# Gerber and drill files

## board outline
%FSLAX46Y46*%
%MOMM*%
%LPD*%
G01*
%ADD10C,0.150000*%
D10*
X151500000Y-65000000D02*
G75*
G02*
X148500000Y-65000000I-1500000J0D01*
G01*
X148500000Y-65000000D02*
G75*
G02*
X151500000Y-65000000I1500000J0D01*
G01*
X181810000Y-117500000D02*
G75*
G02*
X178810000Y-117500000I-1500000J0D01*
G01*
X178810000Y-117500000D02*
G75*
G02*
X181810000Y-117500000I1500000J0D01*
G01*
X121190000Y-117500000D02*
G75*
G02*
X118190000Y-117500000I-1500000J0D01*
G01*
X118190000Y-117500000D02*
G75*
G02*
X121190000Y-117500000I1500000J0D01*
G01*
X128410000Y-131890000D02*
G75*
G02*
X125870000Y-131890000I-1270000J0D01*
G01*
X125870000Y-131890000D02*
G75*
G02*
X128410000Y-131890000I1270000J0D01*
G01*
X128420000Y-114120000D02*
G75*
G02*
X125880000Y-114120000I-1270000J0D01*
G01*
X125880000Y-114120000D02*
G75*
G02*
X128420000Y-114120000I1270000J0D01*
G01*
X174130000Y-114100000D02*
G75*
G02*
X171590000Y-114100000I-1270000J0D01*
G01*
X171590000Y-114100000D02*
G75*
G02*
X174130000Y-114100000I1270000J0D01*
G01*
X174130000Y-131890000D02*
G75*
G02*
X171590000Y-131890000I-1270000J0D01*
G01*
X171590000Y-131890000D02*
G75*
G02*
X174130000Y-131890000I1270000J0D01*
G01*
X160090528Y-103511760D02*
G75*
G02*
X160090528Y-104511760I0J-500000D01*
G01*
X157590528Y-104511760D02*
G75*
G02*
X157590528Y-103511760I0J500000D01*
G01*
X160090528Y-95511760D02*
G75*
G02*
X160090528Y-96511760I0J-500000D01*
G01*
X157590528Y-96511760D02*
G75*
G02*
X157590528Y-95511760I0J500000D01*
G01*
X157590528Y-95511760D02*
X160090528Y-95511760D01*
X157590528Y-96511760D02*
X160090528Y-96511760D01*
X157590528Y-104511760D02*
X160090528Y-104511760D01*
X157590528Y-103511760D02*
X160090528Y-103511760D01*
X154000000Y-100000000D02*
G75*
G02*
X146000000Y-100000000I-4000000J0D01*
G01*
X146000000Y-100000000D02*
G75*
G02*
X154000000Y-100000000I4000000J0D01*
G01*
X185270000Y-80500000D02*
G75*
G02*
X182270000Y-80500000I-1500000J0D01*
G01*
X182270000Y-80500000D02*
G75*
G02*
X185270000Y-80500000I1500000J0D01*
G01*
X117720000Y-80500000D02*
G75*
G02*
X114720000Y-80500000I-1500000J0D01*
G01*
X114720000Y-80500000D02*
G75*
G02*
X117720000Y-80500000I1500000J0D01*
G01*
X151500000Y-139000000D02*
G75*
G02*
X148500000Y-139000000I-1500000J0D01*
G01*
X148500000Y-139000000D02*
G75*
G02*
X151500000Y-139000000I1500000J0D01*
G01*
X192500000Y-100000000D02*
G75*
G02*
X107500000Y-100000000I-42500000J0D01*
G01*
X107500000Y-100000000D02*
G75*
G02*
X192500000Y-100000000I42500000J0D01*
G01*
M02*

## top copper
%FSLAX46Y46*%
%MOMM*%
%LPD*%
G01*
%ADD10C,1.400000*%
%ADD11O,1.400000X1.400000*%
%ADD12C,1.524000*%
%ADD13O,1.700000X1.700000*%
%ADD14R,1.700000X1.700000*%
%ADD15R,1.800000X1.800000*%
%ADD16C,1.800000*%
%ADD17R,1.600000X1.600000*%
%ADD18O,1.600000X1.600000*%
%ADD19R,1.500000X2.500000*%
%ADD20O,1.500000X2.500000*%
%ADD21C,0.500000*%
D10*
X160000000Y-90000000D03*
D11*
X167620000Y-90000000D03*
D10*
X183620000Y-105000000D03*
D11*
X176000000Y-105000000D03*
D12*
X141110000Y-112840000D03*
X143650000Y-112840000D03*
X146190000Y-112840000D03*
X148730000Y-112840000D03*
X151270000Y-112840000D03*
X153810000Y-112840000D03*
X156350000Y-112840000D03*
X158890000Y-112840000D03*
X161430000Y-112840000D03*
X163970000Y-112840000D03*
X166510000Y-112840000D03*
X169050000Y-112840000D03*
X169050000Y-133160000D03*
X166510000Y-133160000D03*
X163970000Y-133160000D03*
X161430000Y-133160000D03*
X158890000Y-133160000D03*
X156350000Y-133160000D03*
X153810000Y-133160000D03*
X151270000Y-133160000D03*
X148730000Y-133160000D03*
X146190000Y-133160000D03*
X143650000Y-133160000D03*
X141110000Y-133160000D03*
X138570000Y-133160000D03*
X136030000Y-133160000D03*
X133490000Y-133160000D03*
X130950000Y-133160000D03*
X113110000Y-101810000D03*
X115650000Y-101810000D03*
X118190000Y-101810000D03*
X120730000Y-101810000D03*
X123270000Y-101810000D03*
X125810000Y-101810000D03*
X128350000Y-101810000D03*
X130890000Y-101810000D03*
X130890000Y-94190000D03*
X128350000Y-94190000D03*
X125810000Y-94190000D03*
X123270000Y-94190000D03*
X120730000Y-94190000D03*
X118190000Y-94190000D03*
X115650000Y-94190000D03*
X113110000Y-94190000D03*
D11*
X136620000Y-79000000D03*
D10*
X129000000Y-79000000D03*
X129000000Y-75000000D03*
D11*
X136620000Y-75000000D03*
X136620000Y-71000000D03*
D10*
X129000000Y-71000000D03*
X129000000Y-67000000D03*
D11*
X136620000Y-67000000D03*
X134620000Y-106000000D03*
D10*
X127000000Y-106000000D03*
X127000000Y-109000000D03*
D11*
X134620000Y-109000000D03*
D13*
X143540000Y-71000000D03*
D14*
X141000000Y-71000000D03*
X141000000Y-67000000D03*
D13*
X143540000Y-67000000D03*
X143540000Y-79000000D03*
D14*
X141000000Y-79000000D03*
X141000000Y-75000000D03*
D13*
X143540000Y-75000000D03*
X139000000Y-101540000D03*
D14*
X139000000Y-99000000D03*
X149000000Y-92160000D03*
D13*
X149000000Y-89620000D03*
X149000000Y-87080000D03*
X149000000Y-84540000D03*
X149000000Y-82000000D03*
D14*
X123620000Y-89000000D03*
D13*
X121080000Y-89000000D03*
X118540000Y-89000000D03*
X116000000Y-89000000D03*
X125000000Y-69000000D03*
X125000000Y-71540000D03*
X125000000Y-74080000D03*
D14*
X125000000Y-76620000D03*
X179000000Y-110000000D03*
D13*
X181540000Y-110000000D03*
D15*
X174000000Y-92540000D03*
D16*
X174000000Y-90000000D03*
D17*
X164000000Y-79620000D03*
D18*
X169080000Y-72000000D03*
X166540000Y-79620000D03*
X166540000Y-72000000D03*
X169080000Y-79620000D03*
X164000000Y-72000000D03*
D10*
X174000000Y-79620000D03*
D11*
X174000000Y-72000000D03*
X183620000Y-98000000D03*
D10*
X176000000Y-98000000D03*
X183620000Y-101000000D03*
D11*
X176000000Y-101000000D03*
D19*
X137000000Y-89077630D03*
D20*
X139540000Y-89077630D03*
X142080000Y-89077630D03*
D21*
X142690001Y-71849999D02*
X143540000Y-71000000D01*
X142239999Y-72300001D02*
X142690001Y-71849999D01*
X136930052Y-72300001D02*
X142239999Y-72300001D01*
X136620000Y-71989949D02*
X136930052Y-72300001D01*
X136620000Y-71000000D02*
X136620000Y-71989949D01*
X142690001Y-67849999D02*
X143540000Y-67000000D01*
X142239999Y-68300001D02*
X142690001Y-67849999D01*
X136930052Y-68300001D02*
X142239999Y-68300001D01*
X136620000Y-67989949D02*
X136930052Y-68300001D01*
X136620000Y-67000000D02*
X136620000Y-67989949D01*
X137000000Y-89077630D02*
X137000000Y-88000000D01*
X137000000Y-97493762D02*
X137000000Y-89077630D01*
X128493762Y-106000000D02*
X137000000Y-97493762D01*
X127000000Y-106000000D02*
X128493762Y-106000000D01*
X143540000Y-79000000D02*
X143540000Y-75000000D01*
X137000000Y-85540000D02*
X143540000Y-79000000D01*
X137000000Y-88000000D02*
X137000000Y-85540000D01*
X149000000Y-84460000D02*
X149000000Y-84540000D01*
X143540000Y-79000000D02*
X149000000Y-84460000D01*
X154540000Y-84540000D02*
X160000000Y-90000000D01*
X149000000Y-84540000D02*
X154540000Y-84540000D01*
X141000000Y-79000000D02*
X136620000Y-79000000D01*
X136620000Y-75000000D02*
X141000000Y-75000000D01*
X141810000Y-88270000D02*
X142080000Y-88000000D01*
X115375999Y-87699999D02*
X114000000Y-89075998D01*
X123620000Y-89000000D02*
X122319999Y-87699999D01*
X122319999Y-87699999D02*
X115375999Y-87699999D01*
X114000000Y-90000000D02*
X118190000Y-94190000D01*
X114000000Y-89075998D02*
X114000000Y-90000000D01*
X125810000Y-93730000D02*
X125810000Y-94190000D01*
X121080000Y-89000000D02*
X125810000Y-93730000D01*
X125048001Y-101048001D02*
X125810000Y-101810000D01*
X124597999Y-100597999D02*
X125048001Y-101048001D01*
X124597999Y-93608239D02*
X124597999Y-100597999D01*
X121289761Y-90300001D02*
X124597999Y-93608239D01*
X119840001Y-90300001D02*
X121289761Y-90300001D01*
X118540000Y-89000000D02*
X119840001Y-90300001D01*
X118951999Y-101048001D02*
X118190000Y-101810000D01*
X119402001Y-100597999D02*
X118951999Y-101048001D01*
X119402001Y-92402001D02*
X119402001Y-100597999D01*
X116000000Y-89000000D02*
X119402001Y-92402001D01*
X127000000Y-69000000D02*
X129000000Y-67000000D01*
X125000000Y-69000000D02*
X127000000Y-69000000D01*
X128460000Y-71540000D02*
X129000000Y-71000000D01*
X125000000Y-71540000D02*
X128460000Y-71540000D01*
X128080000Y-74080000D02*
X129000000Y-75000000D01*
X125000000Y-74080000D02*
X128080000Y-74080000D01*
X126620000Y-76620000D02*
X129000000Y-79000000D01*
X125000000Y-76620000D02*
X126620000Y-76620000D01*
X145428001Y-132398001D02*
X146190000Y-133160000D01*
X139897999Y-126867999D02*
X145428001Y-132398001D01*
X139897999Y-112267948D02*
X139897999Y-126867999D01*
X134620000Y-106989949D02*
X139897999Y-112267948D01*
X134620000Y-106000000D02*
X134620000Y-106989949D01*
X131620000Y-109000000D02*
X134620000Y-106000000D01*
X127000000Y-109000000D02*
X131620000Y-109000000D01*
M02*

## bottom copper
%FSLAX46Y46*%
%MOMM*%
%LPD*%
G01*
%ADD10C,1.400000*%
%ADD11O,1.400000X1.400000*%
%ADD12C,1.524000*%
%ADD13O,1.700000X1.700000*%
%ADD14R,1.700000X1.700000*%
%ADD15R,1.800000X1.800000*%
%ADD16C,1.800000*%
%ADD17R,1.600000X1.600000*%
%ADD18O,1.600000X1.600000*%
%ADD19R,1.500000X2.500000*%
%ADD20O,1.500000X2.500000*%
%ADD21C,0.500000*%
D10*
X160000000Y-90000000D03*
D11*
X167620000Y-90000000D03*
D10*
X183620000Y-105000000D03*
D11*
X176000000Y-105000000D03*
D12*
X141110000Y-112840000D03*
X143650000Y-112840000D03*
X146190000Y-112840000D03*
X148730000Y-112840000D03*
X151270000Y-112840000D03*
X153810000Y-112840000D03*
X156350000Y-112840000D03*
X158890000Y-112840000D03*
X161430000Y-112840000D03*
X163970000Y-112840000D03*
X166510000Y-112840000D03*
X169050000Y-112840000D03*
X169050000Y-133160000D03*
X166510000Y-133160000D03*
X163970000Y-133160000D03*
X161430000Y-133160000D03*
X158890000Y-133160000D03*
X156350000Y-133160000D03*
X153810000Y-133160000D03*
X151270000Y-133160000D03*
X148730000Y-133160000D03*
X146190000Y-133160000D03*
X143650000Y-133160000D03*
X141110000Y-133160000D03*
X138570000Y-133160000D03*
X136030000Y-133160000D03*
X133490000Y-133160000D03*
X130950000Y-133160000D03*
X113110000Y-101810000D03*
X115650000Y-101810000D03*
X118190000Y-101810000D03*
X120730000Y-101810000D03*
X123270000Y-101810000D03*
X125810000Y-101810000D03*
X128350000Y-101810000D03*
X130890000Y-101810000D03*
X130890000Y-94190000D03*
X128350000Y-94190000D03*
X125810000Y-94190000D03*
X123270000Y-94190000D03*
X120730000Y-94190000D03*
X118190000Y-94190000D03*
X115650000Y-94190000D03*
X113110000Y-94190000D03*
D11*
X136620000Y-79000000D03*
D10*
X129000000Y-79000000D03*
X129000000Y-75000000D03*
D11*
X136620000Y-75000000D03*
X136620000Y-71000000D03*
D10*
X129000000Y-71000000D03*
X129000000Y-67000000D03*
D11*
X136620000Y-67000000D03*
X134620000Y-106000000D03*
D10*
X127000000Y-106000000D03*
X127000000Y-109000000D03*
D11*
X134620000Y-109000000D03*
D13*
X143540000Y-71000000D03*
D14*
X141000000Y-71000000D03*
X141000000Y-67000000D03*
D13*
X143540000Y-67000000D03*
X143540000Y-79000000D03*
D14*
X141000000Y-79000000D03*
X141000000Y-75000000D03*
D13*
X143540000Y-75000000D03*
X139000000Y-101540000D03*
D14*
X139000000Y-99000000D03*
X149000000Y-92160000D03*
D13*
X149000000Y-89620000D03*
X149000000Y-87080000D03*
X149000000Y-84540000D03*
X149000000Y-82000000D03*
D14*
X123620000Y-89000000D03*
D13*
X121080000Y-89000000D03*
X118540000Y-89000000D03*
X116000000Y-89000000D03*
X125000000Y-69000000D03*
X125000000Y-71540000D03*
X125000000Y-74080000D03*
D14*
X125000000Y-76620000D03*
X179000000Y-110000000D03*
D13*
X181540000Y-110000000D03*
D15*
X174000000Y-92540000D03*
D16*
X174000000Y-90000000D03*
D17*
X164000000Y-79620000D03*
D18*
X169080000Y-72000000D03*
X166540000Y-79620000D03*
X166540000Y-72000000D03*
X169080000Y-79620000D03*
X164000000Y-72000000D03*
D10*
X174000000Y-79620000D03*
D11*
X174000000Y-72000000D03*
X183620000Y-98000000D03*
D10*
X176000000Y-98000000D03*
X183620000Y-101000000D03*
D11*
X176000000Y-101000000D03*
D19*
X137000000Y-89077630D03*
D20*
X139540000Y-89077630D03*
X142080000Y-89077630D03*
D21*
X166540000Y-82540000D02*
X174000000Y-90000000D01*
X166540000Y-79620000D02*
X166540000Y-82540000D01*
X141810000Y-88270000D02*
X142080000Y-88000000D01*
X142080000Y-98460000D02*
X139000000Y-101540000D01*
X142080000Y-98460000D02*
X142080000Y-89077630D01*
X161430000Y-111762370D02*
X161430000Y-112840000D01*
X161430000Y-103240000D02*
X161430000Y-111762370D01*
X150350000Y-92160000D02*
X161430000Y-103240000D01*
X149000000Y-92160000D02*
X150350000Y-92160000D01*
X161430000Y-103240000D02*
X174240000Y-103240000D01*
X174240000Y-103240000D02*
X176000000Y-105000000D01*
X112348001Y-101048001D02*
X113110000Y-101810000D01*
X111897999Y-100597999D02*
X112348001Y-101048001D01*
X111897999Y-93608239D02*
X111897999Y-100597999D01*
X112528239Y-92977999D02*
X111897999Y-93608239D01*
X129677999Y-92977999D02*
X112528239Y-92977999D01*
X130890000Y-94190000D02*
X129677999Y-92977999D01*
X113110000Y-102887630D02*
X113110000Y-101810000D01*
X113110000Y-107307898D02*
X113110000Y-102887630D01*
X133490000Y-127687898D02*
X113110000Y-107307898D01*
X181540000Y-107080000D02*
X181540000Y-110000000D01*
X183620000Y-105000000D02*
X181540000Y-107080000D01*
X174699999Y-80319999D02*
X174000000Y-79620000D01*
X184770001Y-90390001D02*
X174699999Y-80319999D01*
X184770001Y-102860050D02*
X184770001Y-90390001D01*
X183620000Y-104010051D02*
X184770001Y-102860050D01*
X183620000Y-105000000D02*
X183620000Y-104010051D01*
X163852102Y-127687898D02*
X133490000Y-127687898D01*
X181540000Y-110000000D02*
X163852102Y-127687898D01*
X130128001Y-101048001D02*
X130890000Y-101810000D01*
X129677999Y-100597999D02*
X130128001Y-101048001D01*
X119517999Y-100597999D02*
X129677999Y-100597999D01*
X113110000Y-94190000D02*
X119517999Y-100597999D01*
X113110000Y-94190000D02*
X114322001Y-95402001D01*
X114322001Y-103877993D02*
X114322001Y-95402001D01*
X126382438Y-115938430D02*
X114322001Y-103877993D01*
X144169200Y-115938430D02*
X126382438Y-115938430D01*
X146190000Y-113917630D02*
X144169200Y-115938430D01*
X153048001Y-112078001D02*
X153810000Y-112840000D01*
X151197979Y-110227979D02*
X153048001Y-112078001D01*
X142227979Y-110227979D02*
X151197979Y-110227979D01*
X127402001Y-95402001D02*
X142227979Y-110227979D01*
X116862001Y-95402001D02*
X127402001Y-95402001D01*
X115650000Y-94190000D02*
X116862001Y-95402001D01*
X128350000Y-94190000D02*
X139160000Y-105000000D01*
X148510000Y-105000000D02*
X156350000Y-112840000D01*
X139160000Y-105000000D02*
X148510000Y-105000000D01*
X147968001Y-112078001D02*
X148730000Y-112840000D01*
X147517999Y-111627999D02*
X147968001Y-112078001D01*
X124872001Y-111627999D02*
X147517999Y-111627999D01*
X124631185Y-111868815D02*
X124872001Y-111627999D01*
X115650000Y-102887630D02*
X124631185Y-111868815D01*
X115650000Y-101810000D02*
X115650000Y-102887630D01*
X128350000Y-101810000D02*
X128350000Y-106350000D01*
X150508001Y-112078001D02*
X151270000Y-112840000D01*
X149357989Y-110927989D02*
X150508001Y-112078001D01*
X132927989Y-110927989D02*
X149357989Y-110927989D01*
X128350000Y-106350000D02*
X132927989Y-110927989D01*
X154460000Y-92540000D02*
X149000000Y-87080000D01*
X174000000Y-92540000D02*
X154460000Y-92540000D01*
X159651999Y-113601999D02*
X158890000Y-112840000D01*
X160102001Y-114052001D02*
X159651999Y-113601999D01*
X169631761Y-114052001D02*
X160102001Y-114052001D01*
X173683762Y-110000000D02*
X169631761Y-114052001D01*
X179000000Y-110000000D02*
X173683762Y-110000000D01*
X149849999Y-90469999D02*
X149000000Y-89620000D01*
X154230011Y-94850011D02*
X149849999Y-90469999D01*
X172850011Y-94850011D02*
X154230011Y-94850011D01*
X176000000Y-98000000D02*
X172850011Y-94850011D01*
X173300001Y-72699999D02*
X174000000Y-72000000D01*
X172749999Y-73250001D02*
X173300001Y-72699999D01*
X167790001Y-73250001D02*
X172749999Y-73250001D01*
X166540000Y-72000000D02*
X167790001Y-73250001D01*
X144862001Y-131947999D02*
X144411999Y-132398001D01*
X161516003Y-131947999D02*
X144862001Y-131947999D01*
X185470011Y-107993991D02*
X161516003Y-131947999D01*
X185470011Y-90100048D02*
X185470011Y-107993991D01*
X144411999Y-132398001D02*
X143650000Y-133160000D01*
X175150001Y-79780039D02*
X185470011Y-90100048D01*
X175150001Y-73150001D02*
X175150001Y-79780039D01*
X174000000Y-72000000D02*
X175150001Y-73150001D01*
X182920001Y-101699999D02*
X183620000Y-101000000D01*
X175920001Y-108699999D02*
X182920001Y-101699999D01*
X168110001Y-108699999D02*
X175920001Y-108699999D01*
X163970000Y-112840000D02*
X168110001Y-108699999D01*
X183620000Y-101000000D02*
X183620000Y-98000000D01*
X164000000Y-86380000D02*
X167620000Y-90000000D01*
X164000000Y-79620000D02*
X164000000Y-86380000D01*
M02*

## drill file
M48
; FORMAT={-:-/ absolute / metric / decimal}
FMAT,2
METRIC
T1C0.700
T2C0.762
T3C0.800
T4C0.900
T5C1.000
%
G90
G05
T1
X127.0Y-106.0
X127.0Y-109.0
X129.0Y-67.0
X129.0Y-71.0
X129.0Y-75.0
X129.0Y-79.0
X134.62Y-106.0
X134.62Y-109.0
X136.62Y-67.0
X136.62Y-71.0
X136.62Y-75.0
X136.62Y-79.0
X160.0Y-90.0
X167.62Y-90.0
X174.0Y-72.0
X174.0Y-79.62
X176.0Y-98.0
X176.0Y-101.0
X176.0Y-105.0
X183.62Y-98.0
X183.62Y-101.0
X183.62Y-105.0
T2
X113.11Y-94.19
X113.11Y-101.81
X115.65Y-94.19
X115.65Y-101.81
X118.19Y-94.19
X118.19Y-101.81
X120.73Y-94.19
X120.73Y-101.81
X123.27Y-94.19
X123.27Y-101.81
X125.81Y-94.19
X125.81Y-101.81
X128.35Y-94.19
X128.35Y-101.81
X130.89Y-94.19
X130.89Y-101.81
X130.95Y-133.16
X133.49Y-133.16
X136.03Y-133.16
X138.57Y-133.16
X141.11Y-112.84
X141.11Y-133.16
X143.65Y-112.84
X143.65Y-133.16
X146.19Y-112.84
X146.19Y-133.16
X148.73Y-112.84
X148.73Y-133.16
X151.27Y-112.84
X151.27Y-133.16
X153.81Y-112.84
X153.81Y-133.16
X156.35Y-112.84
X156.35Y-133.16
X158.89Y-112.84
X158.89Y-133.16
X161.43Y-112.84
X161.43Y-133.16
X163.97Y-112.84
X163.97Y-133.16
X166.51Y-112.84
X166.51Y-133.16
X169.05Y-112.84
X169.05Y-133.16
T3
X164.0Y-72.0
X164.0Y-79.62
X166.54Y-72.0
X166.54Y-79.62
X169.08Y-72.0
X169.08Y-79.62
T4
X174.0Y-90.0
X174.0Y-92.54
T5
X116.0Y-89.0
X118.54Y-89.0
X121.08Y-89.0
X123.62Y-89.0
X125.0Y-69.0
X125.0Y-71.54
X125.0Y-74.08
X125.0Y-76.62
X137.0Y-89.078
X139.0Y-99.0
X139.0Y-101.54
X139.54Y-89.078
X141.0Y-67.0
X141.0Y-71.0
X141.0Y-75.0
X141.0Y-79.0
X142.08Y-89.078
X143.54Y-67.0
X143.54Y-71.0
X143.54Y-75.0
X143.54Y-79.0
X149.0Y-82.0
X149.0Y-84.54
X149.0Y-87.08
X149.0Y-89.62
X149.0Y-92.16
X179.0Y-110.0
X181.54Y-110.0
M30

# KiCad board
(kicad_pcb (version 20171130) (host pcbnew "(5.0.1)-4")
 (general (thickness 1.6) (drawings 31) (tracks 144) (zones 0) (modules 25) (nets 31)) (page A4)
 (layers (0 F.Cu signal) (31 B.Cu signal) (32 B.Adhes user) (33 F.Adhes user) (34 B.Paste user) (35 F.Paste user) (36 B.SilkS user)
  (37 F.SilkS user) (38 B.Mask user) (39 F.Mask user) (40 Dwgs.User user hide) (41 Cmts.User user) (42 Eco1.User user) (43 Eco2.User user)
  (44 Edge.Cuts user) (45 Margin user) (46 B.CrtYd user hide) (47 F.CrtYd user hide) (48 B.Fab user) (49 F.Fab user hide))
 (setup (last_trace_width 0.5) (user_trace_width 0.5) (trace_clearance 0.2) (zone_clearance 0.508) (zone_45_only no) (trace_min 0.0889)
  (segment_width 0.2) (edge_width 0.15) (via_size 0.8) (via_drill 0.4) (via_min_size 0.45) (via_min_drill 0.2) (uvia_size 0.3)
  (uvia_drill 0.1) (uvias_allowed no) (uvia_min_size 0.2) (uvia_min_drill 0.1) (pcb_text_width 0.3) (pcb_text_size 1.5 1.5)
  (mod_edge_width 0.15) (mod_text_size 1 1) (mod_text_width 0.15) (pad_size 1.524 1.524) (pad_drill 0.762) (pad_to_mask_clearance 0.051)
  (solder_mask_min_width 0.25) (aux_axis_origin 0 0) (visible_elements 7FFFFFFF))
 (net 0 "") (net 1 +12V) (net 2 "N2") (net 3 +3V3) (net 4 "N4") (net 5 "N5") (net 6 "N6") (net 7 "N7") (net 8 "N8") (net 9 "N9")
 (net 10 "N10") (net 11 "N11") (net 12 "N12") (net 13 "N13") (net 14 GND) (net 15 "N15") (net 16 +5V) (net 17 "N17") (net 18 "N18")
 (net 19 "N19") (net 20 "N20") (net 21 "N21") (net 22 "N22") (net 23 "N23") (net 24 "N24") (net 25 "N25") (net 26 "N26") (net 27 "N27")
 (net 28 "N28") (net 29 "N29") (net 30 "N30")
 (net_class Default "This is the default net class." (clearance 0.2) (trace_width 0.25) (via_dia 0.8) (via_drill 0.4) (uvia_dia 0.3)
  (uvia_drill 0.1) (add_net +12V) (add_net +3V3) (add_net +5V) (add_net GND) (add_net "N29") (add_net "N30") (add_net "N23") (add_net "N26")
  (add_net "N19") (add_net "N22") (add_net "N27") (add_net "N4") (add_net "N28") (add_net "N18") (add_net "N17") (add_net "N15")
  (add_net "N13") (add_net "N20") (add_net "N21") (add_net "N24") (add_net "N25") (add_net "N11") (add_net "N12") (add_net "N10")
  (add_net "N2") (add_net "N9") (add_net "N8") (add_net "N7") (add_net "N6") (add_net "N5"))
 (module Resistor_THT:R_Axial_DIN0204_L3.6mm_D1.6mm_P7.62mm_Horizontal (layer F.Cu) (at 160 90)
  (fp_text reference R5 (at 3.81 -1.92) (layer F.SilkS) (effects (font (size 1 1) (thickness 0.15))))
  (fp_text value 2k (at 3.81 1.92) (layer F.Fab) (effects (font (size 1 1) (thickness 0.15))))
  (pad 1 thru_hole circle (at 0 0) (size 1.4 1.4) (drill 0.7) (layers *.Cu *.Mask) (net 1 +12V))
  (pad 2 thru_hole oval (at 7.62 0) (size 1.4 1.4) (drill 0.7) (layers *.Cu *.Mask) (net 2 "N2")))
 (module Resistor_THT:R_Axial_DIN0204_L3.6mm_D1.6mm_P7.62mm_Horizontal (layer F.Cu) (at 183.62 105 180)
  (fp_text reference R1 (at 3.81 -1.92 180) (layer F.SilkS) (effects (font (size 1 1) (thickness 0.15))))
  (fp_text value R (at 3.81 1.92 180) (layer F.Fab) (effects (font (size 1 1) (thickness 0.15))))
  (pad 1 thru_hole circle (at 0 0 180) (size 1.4 1.4) (drill 0.7) (layers *.Cu *.Mask) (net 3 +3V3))
  (pad 2 thru_hole oval (at 7.62 0 180) (size 1.4 1.4) (drill 0.7) (layers *.Cu *.Mask) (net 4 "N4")))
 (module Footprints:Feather (layer F.Cu) (at 150 123)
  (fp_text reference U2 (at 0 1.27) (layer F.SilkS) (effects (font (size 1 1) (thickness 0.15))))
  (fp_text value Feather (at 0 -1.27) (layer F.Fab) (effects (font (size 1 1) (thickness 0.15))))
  (pad 29 thru_hole circle (at -8.89 -10.16) (size 1.524 1.524) (drill 0.762) (layers *.Cu *.Mask))
  (pad 30 thru_hole circle (at -6.35 -10.16) (size 1.524 1.524) (drill 0.762) (layers *.Cu *.Mask))
  (pad 31 thru_hole circle (at -3.81 -10.16) (size 1.524 1.524) (drill 0.762) (layers *.Cu *.Mask))
  (pad 13 thru_hole circle (at -1.27 -10.16) (size 1.524 1.524) (drill 0.762) (layers *.Cu *.Mask) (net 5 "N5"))
  (pad 12 thru_hole circle (at 1.27 -10.16) (size 1.524 1.524) (drill 0.762) (layers *.Cu *.Mask) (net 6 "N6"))
  (pad 11 thru_hole circle (at 3.81 -10.16) (size 1.524 1.524) (drill 0.762) (layers *.Cu *.Mask) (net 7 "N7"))
  (pad 10 thru_hole circle (at 6.35 -10.16) (size 1.524 1.524) (drill 0.762) (layers *.Cu *.Mask) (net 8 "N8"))
  (pad 9 thru_hole circle (at 8.89 -10.16) (size 1.524 1.524) (drill 0.762) (layers *.Cu *.Mask) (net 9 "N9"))
  (pad 6 thru_hole circle (at 11.43 -10.16) (size 1.524 1.524) (drill 0.762) (layers *.Cu *.Mask) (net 4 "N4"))
  (pad 5 thru_hole circle (at 13.97 -10.16) (size 1.524 1.524) (drill 0.762) (layers *.Cu *.Mask) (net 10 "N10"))
  (pad 21 thru_hole circle (at 16.51 -10.16) (size 1.524 1.524) (drill 0.762) (layers *.Cu *.Mask))
  (pad 20 thru_hole circle (at 19.05 -10.16) (size 1.524 1.524) (drill 0.762) (layers *.Cu *.Mask))
  (pad 2 thru_hole circle (at 19.05 10.16) (size 1.524 1.524) (drill 0.762) (layers *.Cu *.Mask))
  (pad 1 thru_hole circle (at 16.51 10.16) (size 1.524 1.524) (drill 0.762) (layers *.Cu *.Mask))
  (pad 0 thru_hole circle (at 13.97 10.16) (size 1.524 1.524) (drill 0.762) (layers *.Cu *.Mask))
  (pad 22 thru_hole circle (at 11.43 10.16) (size 1.524 1.524) (drill 0.762) (layers *.Cu *.Mask))
  (pad 23 thru_hole circle (at 8.89 10.16) (size 1.524 1.524) (drill 0.762) (layers *.Cu *.Mask))
  (pad 24 thru_hole circle (at 6.35 10.16) (size 1.524 1.524) (drill 0.762) (layers *.Cu *.Mask))
  (pad 19 thru_hole circle (at 3.81 10.16) (size 1.524 1.524) (drill 0.762) (layers *.Cu *.Mask))
  (pad 18 thru_hole circle (at 1.27 10.16) (size 1.524 1.524) (drill 0.762) (layers *.Cu *.Mask))
  (pad 17 thru_hole circle (at -1.27 10.16) (size 1.524 1.524) (drill 0.762) (layers *.Cu *.Mask))
  (pad 16 thru_hole circle (at -3.81 10.16) (size 1.524 1.524) (drill 0.762) (layers *.Cu *.Mask) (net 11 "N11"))
  (pad 15 thru_hole circle (at -6.35 10.16) (size 1.524 1.524) (drill 0.762) (layers *.Cu *.Mask) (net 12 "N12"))
  (pad 14 thru_hole circle (at -8.89 10.16) (size 1.524 1.524) (drill 0.762) (layers *.Cu *.Mask))
  (pad 28 thru_hole circle (at -11.43 10.16) (size 1.524 1.524) (drill 0.762) (layers *.Cu *.Mask))
  (pad 27 thru_hole circle (at -13.97 10.16) (size 1.524 1.524) (drill 0.762) (layers *.Cu *.Mask))
  (pad 26 thru_hole circle (at -16.51 10.16) (size 1.524 1.524) (drill 0.762) (layers *.Cu *.Mask))
  (pad 25 thru_hole circle (at -19.05 10.16) (size 1.524 1.524) (drill 0.762) (layers *.Cu *.Mask)))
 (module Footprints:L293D (layer F.Cu) (at 122 98)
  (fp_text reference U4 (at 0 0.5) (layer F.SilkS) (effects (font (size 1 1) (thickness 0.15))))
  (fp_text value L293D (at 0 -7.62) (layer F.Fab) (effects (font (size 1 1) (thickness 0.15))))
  (pad 1 thru_hole circle (at -8.89 3.81) (size 1.524 1.524) (drill 0.762) (layers *.Cu *.Mask) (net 3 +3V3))
  (pad 2 thru_hole circle (at -6.35 3.81) (size 1.524 1.524) (drill 0.762) (layers *.Cu *.Mask) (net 5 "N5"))
  (pad 3 thru_hole circle (at -3.81 3.81) (size 1.524 1.524) (drill 0.762) (layers *.Cu *.Mask) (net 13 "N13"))
  (pad 4 thru_hole circle (at -1.27 3.81) (size 1.524 1.524) (drill 0.762) (layers *.Cu *.Mask) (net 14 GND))
  (pad 5 thru_hole circle (at 1.27 3.81) (size 1.524 1.524) (drill 0.762) (layers *.Cu *.Mask))
  (pad 6 thru_hole circle (at 3.81 3.81) (size 1.524 1.524) (drill 0.762) (layers *.Cu *.Mask) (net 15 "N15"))
  (pad 7 thru_hole circle (at 6.35 3.81) (size 1.524 1.524) (drill 0.762) (layers *.Cu *.Mask) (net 6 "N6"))
  (pad 8 thru_hole circle (at 8.89 3.81) (size 1.524 1.524) (drill 0.762) (layers *.Cu *.Mask) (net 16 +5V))
  (pad 9 thru_hole circle (at 8.89 -3.81) (size 1.524 1.524) (drill 0.762) (layers *.Cu *.Mask) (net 3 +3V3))
  (pad 10 thru_hole circle (at 6.35 -3.81) (size 1.524 1.524) (drill 0.762) (layers *.Cu *.Mask) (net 8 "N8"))
  (pad 11 thru_hole circle (at 3.81 -3.81) (size 1.524 1.524) (drill 0.762) (layers *.Cu *.Mask) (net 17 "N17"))
  (pad 12 thru_hole circle (at 1.27 -3.81) (size 1.524 1.524) (drill 0.762) (layers *.Cu *.Mask) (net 14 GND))
  (pad 13 thru_hole circle (at -1.27 -3.81) (size 1.524 1.524) (drill 0.762) (layers *.Cu *.Mask) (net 14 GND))
  (pad 14 thru_hole circle (at -3.81 -3.81) (size 1.524 1.524) (drill 0.762) (layers *.Cu *.Mask) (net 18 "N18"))
  (pad 15 thru_hole circle (at -6.35 -3.81) (size 1.524 1.524) (drill 0.762) (layers *.Cu *.Mask) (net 7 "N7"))
  (pad 16 thru_hole circle (at -8.89 -3.81) (size 1.524 1.524) (drill 0.762) (layers *.Cu *.Mask) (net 16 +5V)))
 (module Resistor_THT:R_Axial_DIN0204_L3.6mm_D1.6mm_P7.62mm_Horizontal (layer F.Cu) (at 129 79)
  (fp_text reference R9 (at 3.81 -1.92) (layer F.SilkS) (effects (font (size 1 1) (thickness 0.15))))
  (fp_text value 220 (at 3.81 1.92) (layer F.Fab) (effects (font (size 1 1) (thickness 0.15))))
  (pad 2 thru_hole oval (at 7.62 0) (size 1.4 1.4) (drill 0.7) (layers *.Cu *.Mask) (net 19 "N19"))
  (pad 1 thru_hole circle (at 0 0) (size 1.4 1.4) (drill 0.7) (layers *.Cu *.Mask) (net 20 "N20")))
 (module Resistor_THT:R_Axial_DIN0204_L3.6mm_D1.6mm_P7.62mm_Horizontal (layer F.Cu) (at 129 75)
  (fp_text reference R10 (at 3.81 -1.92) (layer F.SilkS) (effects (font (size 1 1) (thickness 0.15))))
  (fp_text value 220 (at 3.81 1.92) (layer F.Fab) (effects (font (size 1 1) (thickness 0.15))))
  (pad 1 thru_hole circle (at 0 0) (size 1.4 1.4) (drill 0.7) (layers *.Cu *.Mask) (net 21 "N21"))
  (pad 2 thru_hole oval (at 7.62 0) (size 1.4 1.4) (drill 0.7) (layers *.Cu *.Mask) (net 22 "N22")))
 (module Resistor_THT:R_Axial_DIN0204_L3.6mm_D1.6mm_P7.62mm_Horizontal (layer F.Cu) (at 129 71)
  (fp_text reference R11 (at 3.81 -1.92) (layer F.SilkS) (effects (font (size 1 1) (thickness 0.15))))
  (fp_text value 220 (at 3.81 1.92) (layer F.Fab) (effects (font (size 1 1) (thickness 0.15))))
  (pad 2 thru_hole oval (at 7.62 0) (size 1.4 1.4) (drill 0.7) (layers *.Cu *.Mask) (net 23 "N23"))
  (pad 1 thru_hole circle (at 0 0) (size 1.4 1.4) (drill 0.7) (layers *.Cu *.Mask) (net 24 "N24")))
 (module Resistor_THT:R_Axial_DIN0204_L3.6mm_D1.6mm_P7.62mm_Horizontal (layer F.Cu) (at 129 67)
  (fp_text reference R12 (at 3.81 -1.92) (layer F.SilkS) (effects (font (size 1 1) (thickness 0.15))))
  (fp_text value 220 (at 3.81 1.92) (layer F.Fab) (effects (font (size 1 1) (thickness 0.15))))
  (pad 1 thru_hole circle (at 0 0) (size 1.4 1.4) (drill 0.7) (layers *.Cu *.Mask) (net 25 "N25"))
  (pad 2 thru_hole oval (at 7.62 0) (size 1.4 1.4) (drill 0.7) (layers *.Cu *.Mask) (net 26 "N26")))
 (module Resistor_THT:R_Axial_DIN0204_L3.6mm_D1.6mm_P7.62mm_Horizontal (layer F.Cu) (at 127 106)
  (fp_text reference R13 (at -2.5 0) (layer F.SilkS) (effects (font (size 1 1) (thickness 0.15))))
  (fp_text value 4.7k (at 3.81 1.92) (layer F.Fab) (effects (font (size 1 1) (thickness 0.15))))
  (pad 2 thru_hole oval (at 7.62 0) (size 1.4 1.4) (drill 0.7) (layers *.Cu *.Mask) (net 11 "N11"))
  (pad 1 thru_hole circle (at 0 0) (size 1.4 1.4) (drill 0.7) (layers *.Cu *.Mask) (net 1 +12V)))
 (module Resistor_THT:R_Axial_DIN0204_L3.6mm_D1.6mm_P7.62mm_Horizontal (layer F.Cu) (at 127 109)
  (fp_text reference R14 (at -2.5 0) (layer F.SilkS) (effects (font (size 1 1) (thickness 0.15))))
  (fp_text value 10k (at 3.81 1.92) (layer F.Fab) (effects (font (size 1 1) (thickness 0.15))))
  (pad 1 thru_hole circle (at 0 0) (size 1.4 1.4) (drill 0.7) (layers *.Cu *.Mask) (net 11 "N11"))
  (pad 2 thru_hole oval (at 7.62 0) (size 1.4 1.4) (drill 0.7) (layers *.Cu *.Mask) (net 14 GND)))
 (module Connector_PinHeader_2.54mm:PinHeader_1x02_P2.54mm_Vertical (layer F.Cu) (at 141 71 90)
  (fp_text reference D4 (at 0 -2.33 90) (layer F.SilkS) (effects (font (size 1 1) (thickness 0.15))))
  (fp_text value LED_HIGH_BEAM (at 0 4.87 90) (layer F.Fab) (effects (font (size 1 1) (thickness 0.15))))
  (pad 2 thru_hole oval (at 0 2.54 90) (size 1.7 1.7) (drill 1) (layers *.Cu *.Mask) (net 23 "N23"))
  (pad 1 thru_hole rect (at 0 0 90) (size 1.7 1.7) (drill 1) (layers *.Cu *.Mask) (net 14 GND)))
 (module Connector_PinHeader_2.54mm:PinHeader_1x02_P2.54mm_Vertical (layer F.Cu) (at 141 67 90)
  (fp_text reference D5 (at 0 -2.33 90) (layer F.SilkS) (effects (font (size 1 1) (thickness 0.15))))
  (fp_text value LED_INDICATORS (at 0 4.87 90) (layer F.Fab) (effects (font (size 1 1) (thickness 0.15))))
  (pad 1 thru_hole rect (at 0 0 90) (size 1.7 1.7) (drill 1) (layers *.Cu *.Mask) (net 14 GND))
  (pad 2 thru_hole oval (at 0 2.54 90) (size 1.7 1.7) (drill 1) (layers *.Cu *.Mask) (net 26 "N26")))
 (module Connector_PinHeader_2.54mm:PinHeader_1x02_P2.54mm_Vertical (layer F.Cu) (at 141 79 90)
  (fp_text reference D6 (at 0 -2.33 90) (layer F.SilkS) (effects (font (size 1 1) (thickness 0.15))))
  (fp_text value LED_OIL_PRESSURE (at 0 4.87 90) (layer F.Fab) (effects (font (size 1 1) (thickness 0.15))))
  (pad 2 thru_hole oval (at 0 2.54 90) (size 1.7 1.7) (drill 1) (layers *.Cu *.Mask) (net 1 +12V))
  (pad 1 thru_hole rect (at 0 0 90) (size 1.7 1.7) (drill 1) (layers *.Cu *.Mask) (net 19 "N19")))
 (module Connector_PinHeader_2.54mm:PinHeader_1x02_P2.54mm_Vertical (layer F.Cu) (at 141 75 90)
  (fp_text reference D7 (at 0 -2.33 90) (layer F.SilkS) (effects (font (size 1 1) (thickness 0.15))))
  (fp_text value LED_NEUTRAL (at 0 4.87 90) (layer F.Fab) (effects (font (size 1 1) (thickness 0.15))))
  (pad 1 thru_hole rect (at 0 0 90) (size 1.7 1.7) (drill 1) (layers *.Cu *.Mask) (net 22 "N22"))
  (pad 2 thru_hole oval (at 0 2.54 90) (size 1.7 1.7) (drill 1) (layers *.Cu *.Mask) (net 1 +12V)))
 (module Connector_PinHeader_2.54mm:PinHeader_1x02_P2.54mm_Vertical (layer F.Cu) (at 139 99)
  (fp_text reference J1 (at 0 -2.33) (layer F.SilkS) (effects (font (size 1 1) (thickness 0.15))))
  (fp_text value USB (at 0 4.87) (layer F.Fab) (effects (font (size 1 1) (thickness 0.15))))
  (pad 2 thru_hole oval (at 0 2.54) (size 1.7 1.7) (drill 1) (layers *.Cu *.Mask) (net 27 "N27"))
  (pad 1 thru_hole rect (at 0 0) (size 1.7 1.7) (drill 1) (layers *.Cu *.Mask) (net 14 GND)))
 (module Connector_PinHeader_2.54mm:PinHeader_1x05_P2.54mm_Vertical (layer F.Cu) (at 149 92.16 180)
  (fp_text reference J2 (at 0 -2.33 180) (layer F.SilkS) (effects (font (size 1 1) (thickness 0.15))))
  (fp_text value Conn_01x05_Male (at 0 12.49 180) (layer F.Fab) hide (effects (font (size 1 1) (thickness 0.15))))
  (pad 1 thru_hole rect (at 0 0 180) (size 1.7 1.7) (drill 1) (layers *.Cu *.Mask) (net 4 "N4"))
  (pad 2 thru_hole oval (at 0 2.54 180) (size 1.7 1.7) (drill 1) (layers *.Cu *.Mask) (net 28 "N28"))
  (pad 3 thru_hole oval (at 0 5.08 180) (size 1.7 1.7) (drill 1) (layers *.Cu *.Mask) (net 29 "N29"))
  (pad 4 thru_hole oval (at 0 7.62 180) (size 1.7 1.7) (drill 1) (layers *.Cu *.Mask) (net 1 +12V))
  (pad 5 thru_hole oval (at 0 10.16 180) (size 1.7 1.7) (drill 1) (layers *.Cu *.Mask) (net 14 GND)))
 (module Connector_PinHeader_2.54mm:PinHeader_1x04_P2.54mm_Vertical (layer F.Cu) (at 123.62 89 270)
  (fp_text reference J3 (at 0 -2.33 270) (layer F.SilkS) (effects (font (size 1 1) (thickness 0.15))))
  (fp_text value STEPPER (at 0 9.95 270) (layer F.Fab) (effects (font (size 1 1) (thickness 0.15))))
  (pad 1 thru_hole rect (at 0 0 270) (size 1.7 1.7) (drill 1) (layers *.Cu *.Mask) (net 18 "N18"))
  (pad 2 thru_hole oval (at 0 2.54 270) (size 1.7 1.7) (drill 1) (layers *.Cu *.Mask) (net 17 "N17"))
  (pad 3 thru_hole oval (at 0 5.08 270) (size 1.7 1.7) (drill 1) (layers *.Cu *.Mask) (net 15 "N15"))
  (pad 4 thru_hole oval (at 0 7.62 270) (size 1.7 1.7) (drill 1) (layers *.Cu *.Mask) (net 13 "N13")))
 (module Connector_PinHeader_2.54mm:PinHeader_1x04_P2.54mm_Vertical (layer F.Cu) (at 125 76.62 180)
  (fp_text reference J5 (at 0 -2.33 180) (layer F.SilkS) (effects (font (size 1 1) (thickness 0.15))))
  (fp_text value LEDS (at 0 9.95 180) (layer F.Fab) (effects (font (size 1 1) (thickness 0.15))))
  (pad 4 thru_hole oval (at 0 7.62 180) (size 1.7 1.7) (drill 1) (layers *.Cu *.Mask) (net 25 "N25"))
  (pad 3 thru_hole oval (at 0 5.08 180) (size 1.7 1.7) (drill 1) (layers *.Cu *.Mask) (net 24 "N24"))
  (pad 2 thru_hole oval (at 0 2.54 180) (size 1.7 1.7) (drill 1) (layers *.Cu *.Mask) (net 21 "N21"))
  (pad 1 thru_hole rect (at 0 0 180) (size 1.7 1.7) (drill 1) (layers *.Cu *.Mask) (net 20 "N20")))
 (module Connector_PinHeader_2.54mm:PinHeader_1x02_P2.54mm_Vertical (layer F.Cu) (at 179 110 90)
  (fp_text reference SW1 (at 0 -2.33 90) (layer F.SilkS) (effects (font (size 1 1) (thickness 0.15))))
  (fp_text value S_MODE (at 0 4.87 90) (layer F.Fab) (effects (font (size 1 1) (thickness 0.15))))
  (pad 1 thru_hole rect (at 0 0 90) (size 1.7 1.7) (drill 1) (layers *.Cu *.Mask) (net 9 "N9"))
  (pad 2 thru_hole oval (at 0 2.54 90) (size 1.7 1.7) (drill 1) (layers *.Cu *.Mask) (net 3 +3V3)))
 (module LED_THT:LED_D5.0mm (layer F.Cu) (at 174 92.54 90)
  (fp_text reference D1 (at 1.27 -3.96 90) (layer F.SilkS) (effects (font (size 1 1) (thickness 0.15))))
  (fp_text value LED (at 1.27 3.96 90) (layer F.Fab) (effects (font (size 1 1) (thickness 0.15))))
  (pad 1 thru_hole rect (at 0 0 90) (size 1.8 1.8) (drill 0.9) (layers *.Cu *.Mask) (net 29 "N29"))
  (pad 2 thru_hole circle (at 2.54 0 90) (size 1.8 1.8) (drill 0.9) (layers *.Cu *.Mask) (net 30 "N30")))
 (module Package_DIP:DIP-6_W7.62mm (layer F.Cu) (at 164 79.62 90)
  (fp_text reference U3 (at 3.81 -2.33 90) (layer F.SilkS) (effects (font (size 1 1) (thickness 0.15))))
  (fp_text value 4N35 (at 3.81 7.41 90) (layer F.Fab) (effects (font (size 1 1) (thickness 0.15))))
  (pad 1 thru_hole rect (at 0 0 90) (size 1.6 1.6) (drill 0.8) (layers *.Cu *.Mask) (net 2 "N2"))
  (pad 4 thru_hole oval (at 7.62 5.08 90) (size 1.6 1.6) (drill 0.8) (layers *.Cu *.Mask) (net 14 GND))
  (pad 2 thru_hole oval (at 0 2.54 90) (size 1.6 1.6) (drill 0.8) (layers *.Cu *.Mask) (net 30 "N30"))
  (pad 5 thru_hole oval (at 7.62 2.54 90) (size 1.6 1.6) (drill 0.8) (layers *.Cu *.Mask) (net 12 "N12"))
  (pad 3 thru_hole oval (at 0 5.08 90) (size 1.6 1.6) (drill 0.8) (layers *.Cu *.Mask))
  (pad 6 thru_hole oval (at 7.62 0 90) (size 1.6 1.6) (drill 0.8) (layers *.Cu *.Mask)))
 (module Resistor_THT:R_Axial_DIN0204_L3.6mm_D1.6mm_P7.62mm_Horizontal (layer F.Cu) (at 174 79.62 90)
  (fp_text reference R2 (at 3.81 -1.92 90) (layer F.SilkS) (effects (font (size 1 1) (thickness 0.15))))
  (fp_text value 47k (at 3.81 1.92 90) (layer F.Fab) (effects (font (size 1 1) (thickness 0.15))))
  (pad 1 thru_hole circle (at 0 0 90) (size 1.4 1.4) (drill 0.7) (layers *.Cu *.Mask) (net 3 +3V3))
  (pad 2 thru_hole oval (at 7.62 0 90) (size 1.4 1.4) (drill 0.7) (layers *.Cu *.Mask) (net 12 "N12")))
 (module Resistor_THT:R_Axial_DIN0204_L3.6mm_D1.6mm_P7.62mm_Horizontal (layer F.Cu) (at 176 98)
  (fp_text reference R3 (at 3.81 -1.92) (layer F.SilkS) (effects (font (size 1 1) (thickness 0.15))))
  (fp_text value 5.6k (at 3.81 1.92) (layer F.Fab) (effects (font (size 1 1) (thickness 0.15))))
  (pad 2 thru_hole oval (at 7.62 0) (size 1.4 1.4) (drill 0.7) (layers *.Cu *.Mask) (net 10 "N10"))
  (pad 1 thru_hole circle (at 0 0) (size 1.4 1.4) (drill 0.7) (layers *.Cu *.Mask) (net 28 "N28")))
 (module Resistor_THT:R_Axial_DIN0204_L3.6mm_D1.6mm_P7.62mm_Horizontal (layer F.Cu) (at 183.62 101 180)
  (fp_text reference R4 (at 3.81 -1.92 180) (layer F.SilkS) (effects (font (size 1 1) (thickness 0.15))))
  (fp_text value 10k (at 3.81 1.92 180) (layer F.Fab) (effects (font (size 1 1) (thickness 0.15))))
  (pad 1 thru_hole circle (at 0 0 180) (size 1.4 1.4) (drill 0.7) (layers *.Cu *.Mask) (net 10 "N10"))
  (pad 2 thru_hole oval (at 7.62 0 180) (size 1.4 1.4) (drill 0.7) (layers *.Cu *.Mask) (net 14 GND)))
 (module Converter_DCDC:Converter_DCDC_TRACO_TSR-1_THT (layer F.Cu) (at 137 89.07763)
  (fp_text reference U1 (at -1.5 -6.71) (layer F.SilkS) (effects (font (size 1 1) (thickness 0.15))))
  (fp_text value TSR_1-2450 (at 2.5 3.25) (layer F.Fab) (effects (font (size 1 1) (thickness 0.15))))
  (pad 1 thru_hole rect (at 0 0) (size 1.5 2.5) (drill 1) (layers *.Cu *.Mask) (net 1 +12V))
  (pad 2 thru_hole oval (at 2.54 0) (size 1.5 2.5) (drill 1) (layers *.Cu *.Mask) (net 14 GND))
  (pad 3 thru_hole oval (at 5.08 0) (size 1.5 2.5) (drill 1) (layers *.Cu *.Mask) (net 27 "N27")))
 (gr_circle (center 150 65) (end 151.5 65) (layer Edge.Cuts) (width 0.15))
 (gr_circle (center 180.31 117.5) (end 181.81 117.5) (layer Edge.Cuts) (width 0.15))
 (gr_circle (center 119.69 117.5) (end 121.19 117.5) (layer Edge.Cuts) (width 0.15))
 (gr_circle (center 127.14 131.89) (end 128.41 131.89) (layer Edge.Cuts) (width 0.15))
 (gr_circle (center 127.15 114.12) (end 128.42 114.12) (layer Edge.Cuts) (width 0.15))
 (gr_circle (center 172.86 114.1) (end 174.13 114.1) (layer Edge.Cuts) (width 0.15))
 (gr_circle (center 172.86 131.89) (end 174.13 131.89) (layer Edge.Cuts) (width 0.15))
 (gr_arc (start 160.090528 104.01176) (end 160.090528 104.51176) (angle -180) (layer Edge.Cuts) (width 0.15))
 (gr_arc (start 157.590528 104.01176) (end 157.590528 103.51176) (angle -180) (layer Edge.Cuts) (width 0.15))
 (gr_arc (start 160.090528 96.01176) (end 160.090528 96.51176) (angle -180) (layer Edge.Cuts) (width 0.15))
 (gr_arc (start 157.590528 96.01176) (end 157.590528 95.51176) (angle -180) (layer Edge.Cuts) (width 0.15))
 (gr_line (start 157.590528 95.51176) (end 160.090528 95.51176) (layer Edge.Cuts) (width 0.15))
 (gr_line (start 157.590528 96.51176) (end 160.090528 96.51176) (layer Edge.Cuts) (width 0.15))
 (gr_line (start 157.590528 104.51176) (end 160.090528 104.51176) (layer Edge.Cuts) (width 0.15))
 (gr_line (start 157.590528 103.51176) (end 160.090528 103.51176) (layer Edge.Cuts) (width 0.15))
 (gr_circle (center 150 100) (end 154 100) (layer Edge.Cuts) (width 0.15))
 (gr_circle (center 183.77 80.5) (end 185.27 80.5) (layer Edge.Cuts) (width 0.15))
 (gr_circle (center 116.22 80.5) (end 117.72 80.5) (layer Edge.Cuts) (width 0.15))
 (gr_circle (center 150 139) (end 151.5 139) (layer Edge.Cuts) (width 0.15))
 (gr_circle (center 150 100) (end 192.5 100) (layer Edge.Cuts) (width 0.15))
 (segment (start 166.54 82.54) (end 174 90) (width 0.5) (layer B.Cu) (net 30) (status 20))
 (segment (start 166.54 79.62) (end 166.54 82.54) (width 0.5) (layer B.Cu) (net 30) (status 10))
 (segment (start 142.690001 71.849999) (end 143.54 71) (width 0.5) (layer F.Cu) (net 23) (status 30))
 (segment (start 142.239999 72.300001) (end 142.690001 71.849999) (width 0.5) (layer F.Cu) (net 23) (status 20))
 (segment (start 136.930052 72.300001) (end 142.239999 72.300001) (width 0.5) (layer F.Cu) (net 23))
 (segment (start 136.62 71.989949) (end 136.930052 72.300001) (width 0.5) (layer F.Cu) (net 23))
 (segment (start 136.62 71) (end 136.62 71.989949) (width 0.5) (layer F.Cu) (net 23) (status 10))
 (segment (start 142.690001 67.849999) (end 143.54 67) (width 0.5) (layer F.Cu) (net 26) (status 30))
 (segment (start 142.239999 68.300001) (end 142.690001 67.849999) (width 0.5) (layer F.Cu) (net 26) (status 20))
 (segment (start 136.930052 68.300001) (end 142.239999 68.300001) (width 0.5) (layer F.Cu) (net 26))
 (segment (start 136.62 67.989949) (end 136.930052 68.300001) (width 0.5) (layer F.Cu) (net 26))
 (segment (start 136.62 67) (end 136.62 67.989949) (width 0.5) (layer F.Cu) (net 26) (status 10))
 (segment (start 137 89.07763) (end 137 88) (width 0.5) (layer F.Cu) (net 1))
 (segment (start 137 97.493762) (end 137 89.07763) (width 0.5) (layer F.Cu) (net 1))
 (segment (start 128.493762 106) (end 137 97.493762) (width 0.5) (layer F.Cu) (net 1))
 (segment (start 127 106) (end 128.493762 106) (width 0.5) (layer F.Cu) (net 1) (status 10))
 (segment (start 143.54 79) (end 143.54 75) (width 0.5) (layer F.Cu) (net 1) (status 30))
 (segment (start 137 85.54) (end 143.54 79) (width 0.5) (layer F.Cu) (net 1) (status 20))
 (segment (start 137 88) (end 137 85.54) (width 0.5) (layer F.Cu) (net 1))
 (segment (start 149 84.46) (end 149 84.54) (width 0.5) (layer F.Cu) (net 1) (status 30))
 (segment (start 143.54 79) (end 149 84.46) (width 0.5) (layer F.Cu) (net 1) (status 30))
 (segment (start 154.54 84.54) (end 160 90) (width 0.5) (layer F.Cu) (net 1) (status 20))
 (segment (start 149 84.54) (end 154.54 84.54) (width 0.5) (layer F.Cu) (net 1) (status 10))
 (segment (start 141 79) (end 136.62 79) (width 0.5) (layer F.Cu) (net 19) (status 30))
 (segment (start 136.62 75) (end 141 75) (width 0.5) (layer F.Cu) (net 22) (status 30))
 (segment (start 141.81 88.27) (end 142.08 88) (width 0.5) (layer F.Cu) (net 27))
 (segment (start 141.81 88.27) (end 142.08 88) (width 0.5) (layer B.Cu) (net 27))
 (segment (start 142.08 98.46) (end 139 101.54) (width 0.5) (layer B.Cu) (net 27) (status 20))
 (segment (start 142.08 98.46) (end 142.08 89.07763) (width 0.5) (layer B.Cu) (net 27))
 (segment (start 161.43 111.76237) (end 161.43 112.84) (width 0.5) (layer B.Cu) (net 4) (status 20))
 (segment (start 161.43 103.24) (end 161.43 111.76237) (width 0.5) (layer B.Cu) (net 4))
 (segment (start 150.35 92.16) (end 161.43 103.24) (width 0.5) (layer B.Cu) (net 4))
 (segment (start 149 92.16) (end 150.35 92.16) (width 0.5) (layer B.Cu) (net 4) (status 10))
 (segment (start 161.43 103.24) (end 174.24 103.24) (width 0.5) (layer B.Cu) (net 4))
 (segment (start 174.24 103.24) (end 176 105) (width 0.5) (layer B.Cu) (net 4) (status 20))
 (segment (start 115.375999 87.699999) (end 114 89.075998) (width 0.5) (layer F.Cu) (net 18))
 (segment (start 123.62 89) (end 122.319999 87.699999) (width 0.5) (layer F.Cu) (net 18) (status 10))
 (segment (start 122.319999 87.699999) (end 115.375999 87.699999) (width 0.5) (layer F.Cu) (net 18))
 (segment (start 114 90) (end 118.19 94.19) (width 0.5) (layer F.Cu) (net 18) (status 20))
 (segment (start 114 89.075998) (end 114 90) (width 0.5) (layer F.Cu) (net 18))
 (segment (start 125.81 93.73) (end 125.81 94.19) (width 0.5) (layer F.Cu) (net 17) (status 30))
 (segment (start 121.08 89) (end 125.81 93.73) (width 0.5) (layer F.Cu) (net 17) (status 30))
 (segment (start 125.048001 101.048001) (end 125.81 101.81) (width 0.5) (layer F.Cu) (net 15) (status 20))
 (segment (start 124.597999 100.597999) (end 125.048001 101.048001) (width 0.5) (layer F.Cu) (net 15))
 (segment (start 124.597999 93.608239) (end 124.597999 100.597999) (width 0.5) (layer F.Cu) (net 15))
 (segment (start 121.289761 90.300001) (end 124.597999 93.608239) (width 0.5) (layer F.Cu) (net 15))
 (segment (start 119.840001 90.300001) (end 121.289761 90.300001) (width 0.5) (layer F.Cu) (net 15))
 (segment (start 118.54 89) (end 119.840001 90.300001) (width 0.5) (layer F.Cu) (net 15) (status 10))
 (segment (start 118.951999 101.048001) (end 118.19 101.81) (width 0.5) (layer F.Cu) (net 13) (status 20))
 (segment (start 119.402001 100.597999) (end 118.951999 101.048001) (width 0.5) (layer F.Cu) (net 13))
 (segment (start 119.402001 92.402001) (end 119.402001 100.597999) (width 0.5) (layer F.Cu) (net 13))
 (segment (start 116 89) (end 119.402001 92.402001) (width 0.5) (layer F.Cu) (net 13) (status 10))
 (segment (start 112.348001 101.048001) (end 113.11 101.81) (width 0.5) (layer B.Cu) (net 3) (status 20))
 (segment (start 111.897999 100.597999) (end 112.348001 101.048001) (width 0.5) (layer B.Cu) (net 3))
 (segment (start 111.897999 93.608239) (end 111.897999 100.597999) (width 0.5) (layer B.Cu) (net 3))
 (segment (start 112.528239 92.977999) (end 111.897999 93.608239) (width 0.5) (layer B.Cu) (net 3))
 (segment (start 129.677999 92.977999) (end 112.528239 92.977999) (width 0.5) (layer B.Cu) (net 3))
 (segment (start 130.89 94.19) (end 129.677999 92.977999) (width 0.5) (layer B.Cu) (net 3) (status 10))
 (segment (start 113.11 102.88763) (end 113.11 101.81) (width 0.5) (layer B.Cu) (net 3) (status 20))
 (segment (start 113.11 107.307898) (end 113.11 102.88763) (width 0.5) (layer B.Cu) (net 3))
 (segment (start 133.49 127.687898) (end 113.11 107.307898) (width 0.5) (layer B.Cu) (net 3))
 (segment (start 181.54 107.08) (end 181.54 110) (width 0.5) (layer B.Cu) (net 3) (status 20))
 (segment (start 183.62 105) (end 181.54 107.08) (width 0.5) (layer B.Cu) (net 3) (status 10))
 (segment (start 174.699999 80.319999) (end 174 79.62) (width 0.5) (layer B.Cu) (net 3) (status 20))
 (segment (start 184.770001 90.390001) (end 174.699999 80.319999) (width 0.5) (layer B.Cu) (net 3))
 (segment (start 184.770001 102.86005) (end 184.770001 90.390001) (width 0.5) (layer B.Cu) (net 3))
 (segment (start 183.62 104.010051) (end 184.770001 102.86005) (width 0.5) (layer B.Cu) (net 3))
 (segment (start 183.62 105) (end 183.62 104.010051) (width 0.5) (layer B.Cu) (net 3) (status 10))
 (segment (start 163.852102 127.687898) (end 133.49 127.687898) (width 0.5) (layer B.Cu) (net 3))
 (segment (start 181.54 110) (end 163.852102 127.687898) (width 0.5) (layer B.Cu) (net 3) (status 10))
 (segment (start 130.128001 101.048001) (end 130.89 101.81) (width 0.5) (layer B.Cu) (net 16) (status 20))
 (segment (start 129.677999 100.597999) (end 130.128001 101.048001) (width 0.5) (layer B.Cu) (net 16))
 (segment (start 119.517999 100.597999) (end 129.677999 100.597999) (width 0.5) (layer B.Cu) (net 16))
 (segment (start 113.11 94.19) (end 119.517999 100.597999) (width 0.5) (layer B.Cu) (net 16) (status 10))
 (segment (start 113.11 94.19) (end 114.322001 95.402001) (width 0.5) (layer B.Cu) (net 16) (status 10))
 (segment (start 114.322001 103.877993) (end 114.322001 95.402001) (width 0.5) (layer B.Cu) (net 16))
 (segment (start 126.382438 115.93843) (end 114.322001 103.877993) (width 0.5) (layer B.Cu) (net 16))
 (segment (start 144.1692 115.93843) (end 126.382438 115.93843) (width 0.5) (layer B.Cu) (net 16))
 (segment (start 146.19 113.91763) (end 144.1692 115.93843) (width 0.5) (layer B.Cu) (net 16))
 (segment (start 153.048001 112.078001) (end 153.81 112.84) (width 0.5) (layer B.Cu) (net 7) (status 20))
 (segment (start 151.197979 110.227979) (end 153.048001 112.078001) (width 0.5) (layer B.Cu) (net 7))
 (segment (start 142.227979 110.227979) (end 151.197979 110.227979) (width 0.5) (layer B.Cu) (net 7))
 (segment (start 127.402001 95.402001) (end 142.227979 110.227979) (width 0.5) (layer B.Cu) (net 7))
 (segment (start 116.862001 95.402001) (end 127.402001 95.402001) (width 0.5) (layer B.Cu) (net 7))
 (segment (start 115.65 94.19) (end 116.862001 95.402001) (width 0.5) (layer B.Cu) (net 7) (status 10))
 (segment (start 128.35 94.19) (end 139.16 105) (width 0.5) (layer B.Cu) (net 8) (status 10))
 (segment (start 148.51 105) (end 156.35 112.84) (width 0.5) (layer B.Cu) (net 8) (status 20))
 (segment (start 139.16 105) (end 148.51 105) (width 0.5) (layer B.Cu) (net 8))
 (segment (start 127 69) (end 129 67) (width 0.5) (layer F.Cu) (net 25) (status 20))
 (segment (start 125 69) (end 127 69) (width 0.5) (layer F.Cu) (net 25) (status 10))
 (segment (start 128.46 71.54) (end 129 71) (width 0.5) (layer F.Cu) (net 24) (status 20))
 (segment (start 125 71.54) (end 128.46 71.54) (width 0.5) (layer F.Cu) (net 24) (status 10))
 (segment (start 128.08 74.08) (end 129 75) (width 0.5) (layer F.Cu) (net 21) (status 20))
 (segment (start 125 74.08) (end 128.08 74.08) (width 0.5) (layer F.Cu) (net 21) (status 10))
 (segment (start 126.62 76.62) (end 129 79) (width 0.5) (layer F.Cu) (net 20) (status 20))
 (segment (start 125 76.62) (end 126.62 76.62) (width 0.5) (layer F.Cu) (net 20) (status 10))
 (segment (start 147.968001 112.078001) (end 148.73 112.84) (width 0.5) (layer B.Cu) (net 5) (status 20))
 (segment (start 147.517999 111.627999) (end 147.968001 112.078001) (width 0.5) (layer B.Cu) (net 5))
 (segment (start 124.872001 111.627999) (end 147.517999 111.627999) (width 0.5) (layer B.Cu) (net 5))
 (segment (start 124.631185 111.868815) (end 124.872001 111.627999) (width 0.5) (layer B.Cu) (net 5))
 (segment (start 115.65 102.88763) (end 124.631185 111.868815) (width 0.5) (layer B.Cu) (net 5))
 (segment (start 115.65 101.81) (end 115.65 102.88763) (width 0.5) (layer B.Cu) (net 5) (status 10))
 (segment (start 128.35 101.81) (end 128.35 106.35) (width 0.5) (layer B.Cu) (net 6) (status 10))
 (segment (start 150.508001 112.078001) (end 151.27 112.84) (width 0.5) (layer B.Cu) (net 6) (status 20))
 (segment (start 149.357989 110.927989) (end 150.508001 112.078001) (width 0.5) (layer B.Cu) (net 6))
 (segment (start 132.927989 110.927989) (end 149.357989 110.927989) (width 0.5) (layer B.Cu) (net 6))
 (segment (start 128.35 106.35) (end 132.927989 110.927989) (width 0.5) (layer B.Cu) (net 6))
 (segment (start 145.428001 132.398001) (end 146.19 133.16) (width 0.5) (layer F.Cu) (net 11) (status 20))
 (segment (start 139.897999 126.867999) (end 145.428001 132.398001) (width 0.5) (layer F.Cu) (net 11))
 (segment (start 139.897999 112.267948) (end 139.897999 126.867999) (width 0.5) (layer F.Cu) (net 11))
 (segment (start 134.62 106.989949) (end 139.897999 112.267948) (width 0.5) (layer F.Cu) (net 11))
 (segment (start 134.62 106) (end 134.62 106.989949) (width 0.5) (layer F.Cu) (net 11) (status 10))
 (segment (start 131.62 109) (end 134.62 106) (width 0.5) (layer F.Cu) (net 11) (status 20))
 (segment (start 127 109) (end 131.62 109) (width 0.5) (layer F.Cu) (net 11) (status 10))
 (segment (start 154.46 92.54) (end 149 87.08) (width 0.5) (layer B.Cu) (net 29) (status 20))
 (segment (start 174 92.54) (end 154.46 92.54) (width 0.5) (layer B.Cu) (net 29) (status 10))
 (segment (start 159.651999 113.601999) (end 158.89 112.84) (width 0.5) (layer B.Cu) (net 9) (status 20))
 (segment (start 160.102001 114.052001) (end 159.651999 113.601999) (width 0.5) (layer B.Cu) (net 9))
 (segment (start 169.631761 114.052001) (end 160.102001 114.052001) (width 0.5) (layer B.Cu) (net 9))
 (segment (start 173.683762 110) (end 169.631761 114.052001) (width 0.5) (layer B.Cu) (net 9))
 (segment (start 179 110) (end 173.683762 110) (width 0.5) (layer B.Cu) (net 9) (status 10))
 (segment (start 149.849999 90.469999) (end 149 89.62) (width 0.5) (layer B.Cu) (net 28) (status 30))
 (segment (start 154.230011 94.850011) (end 149.849999 90.469999) (width 0.5) (layer B.Cu) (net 28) (status 20))
 (segment (start 172.850011 94.850011) (end 154.230011 94.850011) (width 0.5) (layer B.Cu) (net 28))
 (segment (start 176 98) (end 172.850011 94.850011) (width 0.5) (layer B.Cu) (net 28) (status 10))
 (segment (start 173.300001 72.699999) (end 174 72) (width 0.5) (layer B.Cu) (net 12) (status 30))
 (segment (start 172.749999 73.250001) (end 173.300001 72.699999) (width 0.5) (layer B.Cu) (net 12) (status 20))
 (segment (start 167.790001 73.250001) (end 172.749999 73.250001) (width 0.5) (layer B.Cu) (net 12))
 (segment (start 166.54 72) (end 167.790001 73.250001) (width 0.5) (layer B.Cu) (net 12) (status 10))
 (segment (start 144.862001 131.947999) (end 144.411999 132.398001) (width 0.5) (layer B.Cu) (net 12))
 (segment (start 161.516003 131.947999) (end 144.862001 131.947999) (width 0.5) (layer B.Cu) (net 12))
 (segment (start 185.470011 107.993991) (end 161.516003 131.947999) (width 0.5) (layer B.Cu) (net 12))
 (segment (start 185.470011 90.100048) (end 185.470011 107.993991) (width 0.5) (layer B.Cu) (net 12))
 (segment (start 144.411999 132.398001) (end 143.65 133.16) (width 0.5) (layer B.Cu) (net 12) (status 20))
 (segment (start 175.150001 79.780039) (end 185.470011 90.100048) (width 0.5) (layer B.Cu) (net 12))
 (segment (start 175.150001 73.150001) (end 175.150001 79.780039) (width 0.5) (layer B.Cu) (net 12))
 (segment (start 174 72) (end 175.150001 73.150001) (width 0.5) (layer B.Cu) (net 12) (status 10))
 (segment (start 182.920001 101.699999) (end 183.62 101) (width 0.5) (layer B.Cu) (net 10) (status 20))
 (segment (start 175.920001 108.699999) (end 182.920001 101.699999) (width 0.5) (layer B.Cu) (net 10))
 (segment (start 168.110001 108.699999) (end 175.920001 108.699999) (width 0.5) (layer B.Cu) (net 10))
 (segment (start 163.97 112.84) (end 168.110001 108.699999) (width 0.5) (layer B.Cu) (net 10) (status 10))
 (segment (start 183.62 101) (end 183.62 98) (width 0.5) (layer B.Cu) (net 10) (status 30))
 (segment (start 164 86.38) (end 167.62 90) (width 0.5) (layer B.Cu) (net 2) (status 20))
 (segment (start 164 79.62) (end 164 86.38) (width 0.5) (layer B.Cu) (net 2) (status 10)))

